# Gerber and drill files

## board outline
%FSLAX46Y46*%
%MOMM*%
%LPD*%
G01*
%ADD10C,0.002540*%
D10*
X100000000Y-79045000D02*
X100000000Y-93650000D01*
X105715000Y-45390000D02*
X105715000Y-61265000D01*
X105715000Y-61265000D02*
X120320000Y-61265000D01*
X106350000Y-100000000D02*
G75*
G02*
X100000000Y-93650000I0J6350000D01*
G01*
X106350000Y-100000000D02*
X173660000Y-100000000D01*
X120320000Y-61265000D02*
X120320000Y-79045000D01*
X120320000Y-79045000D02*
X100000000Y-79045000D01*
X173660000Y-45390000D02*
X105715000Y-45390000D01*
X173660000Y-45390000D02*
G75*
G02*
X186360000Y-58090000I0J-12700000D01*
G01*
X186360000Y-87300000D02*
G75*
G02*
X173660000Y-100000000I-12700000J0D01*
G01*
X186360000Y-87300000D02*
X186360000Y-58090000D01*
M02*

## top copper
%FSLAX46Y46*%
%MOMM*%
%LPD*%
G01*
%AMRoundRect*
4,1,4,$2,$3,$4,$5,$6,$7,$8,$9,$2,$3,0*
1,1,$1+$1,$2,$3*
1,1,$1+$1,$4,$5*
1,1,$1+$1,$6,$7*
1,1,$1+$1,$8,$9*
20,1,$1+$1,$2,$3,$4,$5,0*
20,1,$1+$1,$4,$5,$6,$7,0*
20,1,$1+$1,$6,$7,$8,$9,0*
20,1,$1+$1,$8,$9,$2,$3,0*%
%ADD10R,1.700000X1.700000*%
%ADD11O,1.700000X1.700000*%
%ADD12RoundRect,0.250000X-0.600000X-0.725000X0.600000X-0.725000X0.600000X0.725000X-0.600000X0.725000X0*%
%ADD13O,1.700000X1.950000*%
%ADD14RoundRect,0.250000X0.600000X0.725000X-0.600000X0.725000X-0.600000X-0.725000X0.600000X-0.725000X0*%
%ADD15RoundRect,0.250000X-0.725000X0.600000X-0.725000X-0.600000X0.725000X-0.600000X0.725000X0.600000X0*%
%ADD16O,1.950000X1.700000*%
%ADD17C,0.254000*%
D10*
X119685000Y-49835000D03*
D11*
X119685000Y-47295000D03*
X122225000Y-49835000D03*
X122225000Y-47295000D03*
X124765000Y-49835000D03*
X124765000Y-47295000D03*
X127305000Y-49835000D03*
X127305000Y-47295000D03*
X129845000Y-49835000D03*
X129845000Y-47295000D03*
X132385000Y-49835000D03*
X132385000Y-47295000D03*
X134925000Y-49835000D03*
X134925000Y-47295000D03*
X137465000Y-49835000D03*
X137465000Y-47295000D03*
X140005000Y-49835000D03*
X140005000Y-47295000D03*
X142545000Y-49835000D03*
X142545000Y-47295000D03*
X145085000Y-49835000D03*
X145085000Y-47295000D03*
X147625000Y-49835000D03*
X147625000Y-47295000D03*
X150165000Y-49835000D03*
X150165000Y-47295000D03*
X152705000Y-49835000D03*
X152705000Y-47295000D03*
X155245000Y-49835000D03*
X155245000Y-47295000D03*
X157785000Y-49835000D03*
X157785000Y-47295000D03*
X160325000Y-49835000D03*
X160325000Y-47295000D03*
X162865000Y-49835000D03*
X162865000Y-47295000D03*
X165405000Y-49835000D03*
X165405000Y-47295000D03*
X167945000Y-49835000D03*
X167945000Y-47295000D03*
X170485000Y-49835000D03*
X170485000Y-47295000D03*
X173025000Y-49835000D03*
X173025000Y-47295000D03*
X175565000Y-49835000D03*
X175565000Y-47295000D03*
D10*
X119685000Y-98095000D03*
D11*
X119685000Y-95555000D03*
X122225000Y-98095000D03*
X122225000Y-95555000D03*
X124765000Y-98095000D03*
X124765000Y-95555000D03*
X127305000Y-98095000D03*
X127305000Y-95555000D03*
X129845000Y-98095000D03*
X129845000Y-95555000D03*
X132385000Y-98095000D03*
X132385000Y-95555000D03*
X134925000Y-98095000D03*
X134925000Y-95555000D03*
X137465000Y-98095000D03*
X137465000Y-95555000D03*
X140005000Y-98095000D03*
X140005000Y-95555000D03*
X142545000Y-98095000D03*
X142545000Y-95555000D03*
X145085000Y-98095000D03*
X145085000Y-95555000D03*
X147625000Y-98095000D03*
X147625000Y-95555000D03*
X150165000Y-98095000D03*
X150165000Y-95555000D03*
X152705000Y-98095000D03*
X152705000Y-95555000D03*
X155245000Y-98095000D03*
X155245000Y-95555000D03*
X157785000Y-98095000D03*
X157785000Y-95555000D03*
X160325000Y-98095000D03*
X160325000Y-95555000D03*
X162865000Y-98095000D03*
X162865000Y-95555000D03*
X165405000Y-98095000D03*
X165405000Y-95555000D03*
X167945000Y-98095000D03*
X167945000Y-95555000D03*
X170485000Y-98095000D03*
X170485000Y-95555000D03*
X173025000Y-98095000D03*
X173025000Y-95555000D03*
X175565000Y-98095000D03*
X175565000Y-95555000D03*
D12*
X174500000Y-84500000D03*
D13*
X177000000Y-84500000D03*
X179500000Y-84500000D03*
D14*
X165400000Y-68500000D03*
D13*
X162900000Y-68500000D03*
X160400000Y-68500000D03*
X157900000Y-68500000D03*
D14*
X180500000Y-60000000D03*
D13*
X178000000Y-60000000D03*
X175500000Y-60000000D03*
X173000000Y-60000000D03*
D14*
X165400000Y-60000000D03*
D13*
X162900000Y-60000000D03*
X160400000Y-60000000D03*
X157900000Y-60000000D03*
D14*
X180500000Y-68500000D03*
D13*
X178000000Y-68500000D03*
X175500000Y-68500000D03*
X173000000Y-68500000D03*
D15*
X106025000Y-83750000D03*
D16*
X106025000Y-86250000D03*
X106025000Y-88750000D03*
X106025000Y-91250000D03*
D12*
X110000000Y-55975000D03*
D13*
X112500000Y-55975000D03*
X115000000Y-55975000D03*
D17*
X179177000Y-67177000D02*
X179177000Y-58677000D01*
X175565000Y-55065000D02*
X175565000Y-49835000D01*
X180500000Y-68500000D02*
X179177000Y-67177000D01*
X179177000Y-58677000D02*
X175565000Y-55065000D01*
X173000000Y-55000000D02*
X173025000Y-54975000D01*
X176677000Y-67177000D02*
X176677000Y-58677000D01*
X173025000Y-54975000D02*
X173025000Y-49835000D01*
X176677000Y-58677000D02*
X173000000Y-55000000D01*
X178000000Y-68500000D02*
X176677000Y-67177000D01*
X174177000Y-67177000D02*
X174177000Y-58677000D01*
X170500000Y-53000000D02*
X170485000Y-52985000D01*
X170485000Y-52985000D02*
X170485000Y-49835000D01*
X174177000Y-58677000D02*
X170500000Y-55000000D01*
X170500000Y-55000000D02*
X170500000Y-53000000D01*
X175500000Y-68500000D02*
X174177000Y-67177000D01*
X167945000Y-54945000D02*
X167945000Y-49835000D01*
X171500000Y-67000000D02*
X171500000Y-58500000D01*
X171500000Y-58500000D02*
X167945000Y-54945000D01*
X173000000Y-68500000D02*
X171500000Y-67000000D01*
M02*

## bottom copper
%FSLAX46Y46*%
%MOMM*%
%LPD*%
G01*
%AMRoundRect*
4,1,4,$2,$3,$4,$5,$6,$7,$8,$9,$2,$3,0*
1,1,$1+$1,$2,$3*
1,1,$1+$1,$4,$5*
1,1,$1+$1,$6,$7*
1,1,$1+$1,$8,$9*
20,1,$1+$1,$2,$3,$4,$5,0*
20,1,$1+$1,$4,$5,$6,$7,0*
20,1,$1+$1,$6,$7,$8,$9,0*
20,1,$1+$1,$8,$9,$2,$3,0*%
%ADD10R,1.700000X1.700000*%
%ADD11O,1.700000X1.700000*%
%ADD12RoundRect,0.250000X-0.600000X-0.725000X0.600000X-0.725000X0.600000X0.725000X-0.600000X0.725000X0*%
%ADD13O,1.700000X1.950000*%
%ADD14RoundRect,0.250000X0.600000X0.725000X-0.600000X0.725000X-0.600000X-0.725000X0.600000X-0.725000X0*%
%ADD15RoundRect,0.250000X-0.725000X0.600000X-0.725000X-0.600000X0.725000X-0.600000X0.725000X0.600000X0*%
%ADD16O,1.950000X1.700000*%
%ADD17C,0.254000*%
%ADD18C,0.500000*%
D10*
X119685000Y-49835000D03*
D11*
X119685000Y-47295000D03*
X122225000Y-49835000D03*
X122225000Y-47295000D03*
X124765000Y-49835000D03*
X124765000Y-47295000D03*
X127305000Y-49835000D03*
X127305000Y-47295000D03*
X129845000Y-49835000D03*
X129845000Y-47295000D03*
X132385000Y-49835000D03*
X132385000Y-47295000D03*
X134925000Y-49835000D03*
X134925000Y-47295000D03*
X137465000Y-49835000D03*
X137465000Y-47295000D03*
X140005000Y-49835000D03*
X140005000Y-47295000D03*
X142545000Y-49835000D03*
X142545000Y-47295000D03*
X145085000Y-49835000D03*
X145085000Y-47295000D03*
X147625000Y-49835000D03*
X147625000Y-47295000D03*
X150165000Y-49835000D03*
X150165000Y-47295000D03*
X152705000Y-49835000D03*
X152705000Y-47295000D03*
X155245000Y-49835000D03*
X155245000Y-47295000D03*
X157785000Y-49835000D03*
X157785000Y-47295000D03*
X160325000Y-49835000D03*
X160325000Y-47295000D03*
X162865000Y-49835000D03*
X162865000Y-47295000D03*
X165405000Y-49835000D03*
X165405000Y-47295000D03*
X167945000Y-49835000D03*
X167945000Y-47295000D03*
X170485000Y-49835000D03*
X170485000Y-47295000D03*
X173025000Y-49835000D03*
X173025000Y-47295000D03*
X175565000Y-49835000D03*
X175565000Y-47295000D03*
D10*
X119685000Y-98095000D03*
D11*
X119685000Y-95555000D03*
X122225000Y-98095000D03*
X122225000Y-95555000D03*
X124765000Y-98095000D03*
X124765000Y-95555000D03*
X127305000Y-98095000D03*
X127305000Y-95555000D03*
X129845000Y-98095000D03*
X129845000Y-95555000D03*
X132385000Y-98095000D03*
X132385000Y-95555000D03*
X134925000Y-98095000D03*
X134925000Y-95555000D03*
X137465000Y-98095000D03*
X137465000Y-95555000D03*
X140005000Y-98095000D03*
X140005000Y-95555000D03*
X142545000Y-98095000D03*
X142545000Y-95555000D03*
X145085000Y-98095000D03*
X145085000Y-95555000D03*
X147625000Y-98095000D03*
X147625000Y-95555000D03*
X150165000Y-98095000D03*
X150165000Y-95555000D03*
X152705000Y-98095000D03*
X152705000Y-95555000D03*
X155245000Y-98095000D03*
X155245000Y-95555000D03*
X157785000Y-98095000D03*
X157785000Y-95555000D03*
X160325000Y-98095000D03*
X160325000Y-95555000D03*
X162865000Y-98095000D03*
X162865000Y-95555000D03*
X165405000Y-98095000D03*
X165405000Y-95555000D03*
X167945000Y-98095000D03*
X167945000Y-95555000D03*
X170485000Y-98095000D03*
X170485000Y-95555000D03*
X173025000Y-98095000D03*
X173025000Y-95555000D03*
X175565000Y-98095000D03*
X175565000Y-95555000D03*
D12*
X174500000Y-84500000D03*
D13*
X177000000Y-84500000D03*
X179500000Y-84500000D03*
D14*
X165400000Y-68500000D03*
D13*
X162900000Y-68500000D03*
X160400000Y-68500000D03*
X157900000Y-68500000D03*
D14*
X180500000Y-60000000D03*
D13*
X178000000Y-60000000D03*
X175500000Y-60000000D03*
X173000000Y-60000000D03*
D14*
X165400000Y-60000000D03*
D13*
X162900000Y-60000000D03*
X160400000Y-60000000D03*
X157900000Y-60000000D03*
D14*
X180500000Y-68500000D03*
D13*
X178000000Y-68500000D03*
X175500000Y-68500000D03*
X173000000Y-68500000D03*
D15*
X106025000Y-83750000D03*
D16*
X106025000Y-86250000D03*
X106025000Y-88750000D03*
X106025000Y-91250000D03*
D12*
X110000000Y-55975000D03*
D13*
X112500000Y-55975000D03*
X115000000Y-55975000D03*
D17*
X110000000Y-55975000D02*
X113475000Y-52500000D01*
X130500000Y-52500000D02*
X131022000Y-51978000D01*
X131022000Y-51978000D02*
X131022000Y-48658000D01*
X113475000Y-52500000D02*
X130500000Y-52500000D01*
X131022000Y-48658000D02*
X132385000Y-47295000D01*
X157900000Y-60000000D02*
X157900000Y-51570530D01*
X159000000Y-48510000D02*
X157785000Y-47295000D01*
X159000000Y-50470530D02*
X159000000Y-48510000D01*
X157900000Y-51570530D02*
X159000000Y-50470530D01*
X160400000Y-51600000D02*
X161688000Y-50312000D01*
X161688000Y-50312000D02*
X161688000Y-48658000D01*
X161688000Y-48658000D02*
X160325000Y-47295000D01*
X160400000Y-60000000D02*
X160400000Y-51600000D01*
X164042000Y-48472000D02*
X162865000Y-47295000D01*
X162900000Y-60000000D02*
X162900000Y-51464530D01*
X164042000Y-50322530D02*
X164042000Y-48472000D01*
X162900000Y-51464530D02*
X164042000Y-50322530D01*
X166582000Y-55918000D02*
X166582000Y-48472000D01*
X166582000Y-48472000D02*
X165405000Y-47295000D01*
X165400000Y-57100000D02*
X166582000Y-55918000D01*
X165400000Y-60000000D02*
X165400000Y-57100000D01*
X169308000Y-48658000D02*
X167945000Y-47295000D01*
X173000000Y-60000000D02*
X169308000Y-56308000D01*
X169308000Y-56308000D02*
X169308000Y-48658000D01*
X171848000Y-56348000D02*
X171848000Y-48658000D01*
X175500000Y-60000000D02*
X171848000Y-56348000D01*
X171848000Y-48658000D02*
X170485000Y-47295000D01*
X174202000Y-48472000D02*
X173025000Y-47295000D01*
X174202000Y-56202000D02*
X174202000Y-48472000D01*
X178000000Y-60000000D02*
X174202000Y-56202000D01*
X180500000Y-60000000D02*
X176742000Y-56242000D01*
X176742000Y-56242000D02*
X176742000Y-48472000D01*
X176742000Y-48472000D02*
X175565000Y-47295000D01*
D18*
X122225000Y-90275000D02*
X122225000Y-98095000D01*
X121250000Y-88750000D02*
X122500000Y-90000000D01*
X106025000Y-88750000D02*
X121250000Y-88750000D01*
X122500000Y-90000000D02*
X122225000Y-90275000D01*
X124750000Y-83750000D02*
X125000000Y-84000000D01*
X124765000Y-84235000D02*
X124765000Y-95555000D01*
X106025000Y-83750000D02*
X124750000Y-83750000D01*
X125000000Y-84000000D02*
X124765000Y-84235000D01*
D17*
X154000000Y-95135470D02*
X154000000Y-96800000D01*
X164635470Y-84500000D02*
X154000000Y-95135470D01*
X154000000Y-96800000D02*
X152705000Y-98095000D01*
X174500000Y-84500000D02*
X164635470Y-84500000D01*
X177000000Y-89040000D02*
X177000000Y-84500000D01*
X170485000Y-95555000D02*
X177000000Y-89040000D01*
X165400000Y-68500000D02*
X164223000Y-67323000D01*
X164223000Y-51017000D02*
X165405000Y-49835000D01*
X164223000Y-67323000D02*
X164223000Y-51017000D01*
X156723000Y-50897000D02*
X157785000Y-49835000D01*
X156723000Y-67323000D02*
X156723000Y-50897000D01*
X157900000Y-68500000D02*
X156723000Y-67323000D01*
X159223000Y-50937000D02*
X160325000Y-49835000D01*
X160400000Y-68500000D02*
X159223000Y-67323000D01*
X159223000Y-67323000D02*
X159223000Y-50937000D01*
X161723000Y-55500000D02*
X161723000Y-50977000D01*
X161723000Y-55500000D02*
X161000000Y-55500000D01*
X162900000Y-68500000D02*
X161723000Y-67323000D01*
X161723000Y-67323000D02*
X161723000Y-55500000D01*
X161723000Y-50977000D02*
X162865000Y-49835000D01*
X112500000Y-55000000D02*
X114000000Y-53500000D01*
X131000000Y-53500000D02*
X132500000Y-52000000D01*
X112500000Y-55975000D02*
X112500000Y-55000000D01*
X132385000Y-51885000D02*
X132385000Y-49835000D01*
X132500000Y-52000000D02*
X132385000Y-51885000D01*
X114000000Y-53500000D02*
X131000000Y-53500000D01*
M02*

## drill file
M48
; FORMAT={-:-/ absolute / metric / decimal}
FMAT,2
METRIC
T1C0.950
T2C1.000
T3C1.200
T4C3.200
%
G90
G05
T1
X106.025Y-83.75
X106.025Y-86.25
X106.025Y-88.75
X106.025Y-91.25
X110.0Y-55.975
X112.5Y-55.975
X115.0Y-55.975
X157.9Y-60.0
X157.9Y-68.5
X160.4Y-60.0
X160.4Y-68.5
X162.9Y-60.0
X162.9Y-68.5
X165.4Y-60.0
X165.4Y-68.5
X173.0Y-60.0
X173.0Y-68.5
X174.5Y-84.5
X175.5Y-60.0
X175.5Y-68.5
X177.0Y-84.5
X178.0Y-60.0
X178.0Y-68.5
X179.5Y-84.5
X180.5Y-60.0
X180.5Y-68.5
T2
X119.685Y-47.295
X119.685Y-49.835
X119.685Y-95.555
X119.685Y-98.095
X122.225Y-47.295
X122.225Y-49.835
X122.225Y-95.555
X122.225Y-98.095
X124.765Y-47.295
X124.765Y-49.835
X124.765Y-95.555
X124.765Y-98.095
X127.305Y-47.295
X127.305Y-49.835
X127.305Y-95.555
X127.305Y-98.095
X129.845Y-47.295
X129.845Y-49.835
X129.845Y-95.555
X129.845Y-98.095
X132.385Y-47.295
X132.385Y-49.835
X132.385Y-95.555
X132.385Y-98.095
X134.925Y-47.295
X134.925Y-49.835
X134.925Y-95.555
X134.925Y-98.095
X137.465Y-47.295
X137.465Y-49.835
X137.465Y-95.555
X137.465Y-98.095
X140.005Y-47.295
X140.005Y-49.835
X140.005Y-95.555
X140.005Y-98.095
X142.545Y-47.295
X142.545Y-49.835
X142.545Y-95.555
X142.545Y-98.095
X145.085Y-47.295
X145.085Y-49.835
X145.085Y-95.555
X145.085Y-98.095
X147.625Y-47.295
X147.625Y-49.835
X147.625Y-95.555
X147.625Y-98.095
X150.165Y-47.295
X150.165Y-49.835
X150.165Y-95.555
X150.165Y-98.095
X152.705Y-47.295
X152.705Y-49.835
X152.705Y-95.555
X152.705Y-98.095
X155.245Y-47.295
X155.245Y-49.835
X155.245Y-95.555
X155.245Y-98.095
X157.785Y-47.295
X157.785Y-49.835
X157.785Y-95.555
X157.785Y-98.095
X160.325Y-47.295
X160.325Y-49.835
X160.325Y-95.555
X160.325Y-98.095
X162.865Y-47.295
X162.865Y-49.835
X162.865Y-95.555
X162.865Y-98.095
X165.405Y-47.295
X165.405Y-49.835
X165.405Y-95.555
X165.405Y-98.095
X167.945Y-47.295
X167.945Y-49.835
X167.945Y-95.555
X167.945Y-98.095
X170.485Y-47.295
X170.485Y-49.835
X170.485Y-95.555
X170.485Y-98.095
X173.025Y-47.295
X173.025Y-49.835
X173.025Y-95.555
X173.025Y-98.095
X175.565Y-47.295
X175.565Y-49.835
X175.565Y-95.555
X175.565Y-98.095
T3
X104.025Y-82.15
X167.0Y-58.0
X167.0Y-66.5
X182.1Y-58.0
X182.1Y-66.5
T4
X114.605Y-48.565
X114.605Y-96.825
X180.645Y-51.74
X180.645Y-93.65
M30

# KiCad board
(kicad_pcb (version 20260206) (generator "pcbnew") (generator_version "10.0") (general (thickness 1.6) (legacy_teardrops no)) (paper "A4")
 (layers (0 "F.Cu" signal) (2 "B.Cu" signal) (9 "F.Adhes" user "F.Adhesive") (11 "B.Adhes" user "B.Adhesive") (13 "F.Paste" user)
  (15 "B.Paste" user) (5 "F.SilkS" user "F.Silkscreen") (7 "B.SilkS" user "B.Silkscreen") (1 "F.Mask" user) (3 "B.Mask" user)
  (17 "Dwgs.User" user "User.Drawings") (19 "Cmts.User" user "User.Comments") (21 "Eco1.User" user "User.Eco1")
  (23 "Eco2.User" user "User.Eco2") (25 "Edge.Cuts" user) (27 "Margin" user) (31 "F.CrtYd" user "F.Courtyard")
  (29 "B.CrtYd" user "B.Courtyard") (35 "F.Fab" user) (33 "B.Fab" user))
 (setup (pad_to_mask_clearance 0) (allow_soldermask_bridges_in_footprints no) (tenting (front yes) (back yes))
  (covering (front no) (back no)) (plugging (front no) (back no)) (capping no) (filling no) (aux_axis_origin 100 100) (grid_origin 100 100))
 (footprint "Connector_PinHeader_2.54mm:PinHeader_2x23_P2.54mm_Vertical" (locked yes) (layer "F.Cu") (at 119.685 49.835 90)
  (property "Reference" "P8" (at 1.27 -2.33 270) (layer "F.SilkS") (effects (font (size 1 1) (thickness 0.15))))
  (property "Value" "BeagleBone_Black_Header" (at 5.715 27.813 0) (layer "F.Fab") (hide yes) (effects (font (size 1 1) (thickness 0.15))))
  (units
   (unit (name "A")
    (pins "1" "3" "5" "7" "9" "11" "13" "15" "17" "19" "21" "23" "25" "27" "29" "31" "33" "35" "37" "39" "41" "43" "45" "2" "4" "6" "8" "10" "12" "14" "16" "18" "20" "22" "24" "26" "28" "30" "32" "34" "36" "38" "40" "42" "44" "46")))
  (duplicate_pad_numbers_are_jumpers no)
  (pad "1" thru_hole rect (at 0 0 90) (size 1.7 1.7) (drill 1) (layers "*.Cu" "*.Mask") (remove_unused_layers no) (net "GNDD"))
  (pad "2" thru_hole oval (at 2.54 0 90) (size 1.7 1.7) (drill 1) (layers "*.Cu" "*.Mask") (remove_unused_layers no) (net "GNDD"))
  (pad "3" thru_hole oval (at 0 2.54 90) (size 1.7 1.7) (drill 1) (layers "*.Cu" "*.Mask") (remove_unused_layers no)
   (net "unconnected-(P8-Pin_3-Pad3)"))
  (pad "4" thru_hole oval (at 2.54 2.54 90) (size 1.7 1.7) (drill 1) (layers "*.Cu" "*.Mask") (remove_unused_layers no) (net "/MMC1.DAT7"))
  (pad "5" thru_hole oval (at 0 5.08 90) (size 1.7 1.7) (drill 1) (layers "*.Cu" "*.Mask") (remove_unused_layers no)
   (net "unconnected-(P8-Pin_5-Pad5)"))
  (pad "6" thru_hole oval (at 2.54 5.08 90) (size 1.7 1.7) (drill 1) (layers "*.Cu" "*.Mask") (remove_unused_layers no) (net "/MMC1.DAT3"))
  (pad "7" thru_hole oval (at 0 7.62 90) (size 1.7 1.7) (drill 1) (layers "*.Cu" "*.Mask") (remove_unused_layers no)
   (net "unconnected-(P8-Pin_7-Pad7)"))
  (pad "8" thru_hole oval (at 2.54 7.62 90) (size 1.7 1.7) (drill 1) (layers "*.Cu" "*.Mask") (remove_unused_layers no) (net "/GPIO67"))
  (pad "9" thru_hole oval (at 0 10.16 90) (size 1.7 1.7) (drill 1) (layers "*.Cu" "*.Mask") (remove_unused_layers no)
   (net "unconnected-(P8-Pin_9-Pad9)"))
  (pad "10" thru_hole oval (at 2.54 10.16 90) (size 1.7 1.7) (drill 1) (layers "*.Cu" "*.Mask") (remove_unused_layers no) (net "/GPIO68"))
  (pad "11" thru_hole oval (at 0 12.7 90) (size 1.7 1.7) (drill 1) (layers "*.Cu" "*.Mask") (remove_unused_layers no) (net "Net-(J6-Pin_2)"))
  (pad "12" thru_hole oval (at 2.54 12.7 90) (size 1.7 1.7) (drill 1) (layers "*.Cu" "*.Mask") (remove_unused_layers no) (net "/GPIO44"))
  (pad "13" thru_hole oval (at 0 15.24 90) (size 1.7 1.7) (drill 1) (layers "*.Cu" "*.Mask") (remove_unused_layers no)
   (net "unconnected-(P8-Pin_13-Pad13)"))
  (pad "14" thru_hole oval (at 2.54 15.24 90) (size 1.7 1.7) (drill 1) (layers "*.Cu" "*.Mask") (remove_unused_layers no) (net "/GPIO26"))
  (pad "15" thru_hole oval (at 0 17.78 90) (size 1.7 1.7) (drill 1) (layers "*.Cu" "*.Mask") (remove_unused_layers no)
   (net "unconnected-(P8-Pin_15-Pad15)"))
  (pad "16" thru_hole oval (at 2.54 17.78 90) (size 1.7 1.7) (drill 1) (layers "*.Cu" "*.Mask") (remove_unused_layers no) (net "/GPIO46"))
  (pad "17" thru_hole oval (at 0 20.32 90) (size 1.7 1.7) (drill 1) (layers "*.Cu" "*.Mask") (remove_unused_layers no)
   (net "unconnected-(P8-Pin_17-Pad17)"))
  (pad "18" thru_hole oval (at 2.54 20.32 90) (size 1.7 1.7) (drill 1) (layers "*.Cu" "*.Mask") (remove_unused_layers no) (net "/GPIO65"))
  (pad "19" thru_hole oval (at 0 22.86 90) (size 1.7 1.7) (drill 1) (layers "*.Cu" "*.Mask") (remove_unused_layers no)
   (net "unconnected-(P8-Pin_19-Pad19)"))
  (pad "20" thru_hole oval (at 2.54 22.86 90) (size 1.7 1.7) (drill 1) (layers "*.Cu" "*.Mask") (remove_unused_layers no) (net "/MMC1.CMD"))
  (pad "21" thru_hole oval (at 0 25.4 90) (size 1.7 1.7) (drill 1) (layers "*.Cu" "*.Mask") (remove_unused_layers no)
   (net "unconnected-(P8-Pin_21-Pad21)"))
  (pad "22" thru_hole oval (at 2.54 25.4 90) (size 1.7 1.7) (drill 1) (layers "*.Cu" "*.Mask") (remove_unused_layers no) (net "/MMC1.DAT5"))
  (pad "23" thru_hole oval (at 0 27.94 90) (size 1.7 1.7) (drill 1) (layers "*.Cu" "*.Mask") (remove_unused_layers no)
   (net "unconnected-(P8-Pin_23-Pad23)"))
  (pad "24" thru_hole oval (at 2.54 27.94 90) (size 1.7 1.7) (drill 1) (layers "*.Cu" "*.Mask") (remove_unused_layers no) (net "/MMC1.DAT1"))
  (pad "25" thru_hole oval (at 0 30.48 90) (size 1.7 1.7) (drill 1) (layers "*.Cu" "*.Mask") (remove_unused_layers no)
   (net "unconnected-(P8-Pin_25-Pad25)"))
  (pad "26" thru_hole oval (at 2.54 30.48 90) (size 1.7 1.7) (drill 1) (layers "*.Cu" "*.Mask") (remove_unused_layers no) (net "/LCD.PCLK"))
  (pad "27" thru_hole oval (at 0 33.02 90) (size 1.7 1.7) (drill 1) (layers "*.Cu" "*.Mask") (remove_unused_layers no)
   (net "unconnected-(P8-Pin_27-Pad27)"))
  (pad "28" thru_hole oval (at 2.54 33.02 90) (size 1.7 1.7) (drill 1) (layers "*.Cu" "*.Mask") (remove_unused_layers no) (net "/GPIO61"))
  (pad "29" thru_hole oval (at 0 35.56 90) (size 1.7 1.7) (drill 1) (layers "*.Cu" "*.Mask") (remove_unused_layers no)
   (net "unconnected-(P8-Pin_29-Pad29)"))
  (pad "30" thru_hole oval (at 2.54 35.56 90) (size 1.7 1.7) (drill 1) (layers "*.Cu" "*.Mask") (remove_unused_layers no)
   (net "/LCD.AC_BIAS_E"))
  (pad "31" thru_hole oval (at 0 38.1 90) (size 1.7 1.7) (drill 1) (layers "*.Cu" "*.Mask") (remove_unused_layers no) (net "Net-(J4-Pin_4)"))
  (pad "32" thru_hole oval (at 2.54 38.1 90) (size 1.7 1.7) (drill 1) (layers "*.Cu" "*.Mask") (remove_unused_layers no) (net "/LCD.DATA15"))
  (pad "33" thru_hole oval (at 0 40.64 90) (size 1.7 1.7) (drill 1) (layers "*.Cu" "*.Mask") (remove_unused_layers no)
   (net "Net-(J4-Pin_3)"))
  (pad "34" thru_hole oval (at 2.54 40.64 90) (size 1.7 1.7) (drill 1) (layers "*.Cu" "*.Mask") (remove_unused_layers no)
   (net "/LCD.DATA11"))
  (pad "35" thru_hole oval (at 0 43.18 90) (size 1.7 1.7) (drill 1) (layers "*.Cu" "*.Mask") (remove_unused_layers no)
   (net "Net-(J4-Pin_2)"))
  (pad "36" thru_hole oval (at 2.54 43.18 90) (size 1.7 1.7) (drill 1) (layers "*.Cu" "*.Mask") (remove_unused_layers no)
   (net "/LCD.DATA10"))
  (pad "37" thru_hole oval (at 0 45.72 90) (size 1.7 1.7) (drill 1) (layers "*.Cu" "*.Mask") (remove_unused_layers no)
   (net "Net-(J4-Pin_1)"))
  (pad "38" thru_hole oval (at 2.54 45.72 90) (size 1.7 1.7) (drill 1) (layers "*.Cu" "*.Mask") (remove_unused_layers no) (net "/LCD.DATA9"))
  (pad "39" thru_hole oval (at 0 48.26 90) (size 1.7 1.7) (drill 1) (layers "*.Cu" "*.Mask") (remove_unused_layers no)
   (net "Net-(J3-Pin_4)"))
  (pad "40" thru_hole oval (at 2.54 48.26 90) (size 1.7 1.7) (drill 1) (layers "*.Cu" "*.Mask") (remove_unused_layers no) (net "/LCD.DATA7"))
  (pad "41" thru_hole oval (at 0 50.8 90) (size 1.7 1.7) (drill 1) (layers "*.Cu" "*.Mask") (remove_unused_layers no) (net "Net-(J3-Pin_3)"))
  (pad "42" thru_hole oval (at 2.54 50.8 90) (size 1.7 1.7) (drill 1) (layers "*.Cu" "*.Mask") (remove_unused_layers no) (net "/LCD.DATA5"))
  (pad "43" thru_hole oval (at 0 53.34 90) (size 1.7 1.7) (drill 1) (layers "*.Cu" "*.Mask") (remove_unused_layers no)
   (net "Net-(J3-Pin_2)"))
  (pad "44" thru_hole oval (at 2.54 53.34 90) (size 1.7 1.7) (drill 1) (layers "*.Cu" "*.Mask") (remove_unused_layers no) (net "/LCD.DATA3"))
  (pad "45" thru_hole oval (at 0 55.88 90) (size 1.7 1.7) (drill 1) (layers "*.Cu" "*.Mask") (remove_unused_layers no)
   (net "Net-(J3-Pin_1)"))
  (pad "46" thru_hole oval (at 2.54 55.88 90) (size 1.7 1.7) (drill 1) (layers "*.Cu" "*.Mask") (remove_unused_layers no) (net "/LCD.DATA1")))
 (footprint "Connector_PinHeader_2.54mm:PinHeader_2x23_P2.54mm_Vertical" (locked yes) (layer "F.Cu") (at 119.685 98.095 90)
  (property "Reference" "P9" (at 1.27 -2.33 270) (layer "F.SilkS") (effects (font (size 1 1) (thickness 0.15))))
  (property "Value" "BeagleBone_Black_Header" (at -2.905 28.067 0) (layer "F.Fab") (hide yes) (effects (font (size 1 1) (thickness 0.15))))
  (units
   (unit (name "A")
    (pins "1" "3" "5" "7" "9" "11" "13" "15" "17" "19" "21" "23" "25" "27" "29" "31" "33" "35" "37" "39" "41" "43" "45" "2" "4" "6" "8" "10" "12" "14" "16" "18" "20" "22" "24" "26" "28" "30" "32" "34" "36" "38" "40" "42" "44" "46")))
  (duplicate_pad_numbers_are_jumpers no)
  (pad "1" thru_hole rect (at 0 0 90) (size 1.7 1.7) (drill 1) (layers "*.Cu" "*.Mask") (remove_unused_layers no) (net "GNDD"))
  (pad "2" thru_hole oval (at 2.54 0 90) (size 1.7 1.7) (drill 1) (layers "*.Cu" "*.Mask") (remove_unused_layers no) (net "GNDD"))
  (pad "3" thru_hole oval (at 0 2.54 90) (size 1.7 1.7) (drill 1) (layers "*.Cu" "*.Mask") (remove_unused_layers no) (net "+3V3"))
  (pad "4" thru_hole oval (at 2.54 2.54 90) (size 1.7 1.7) (drill 1) (layers "*.Cu" "*.Mask") (remove_unused_layers no) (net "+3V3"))
  (pad "5" thru_hole oval (at 0 5.08 90) (size 1.7 1.7) (drill 1) (layers "*.Cu" "*.Mask") (remove_unused_layers no) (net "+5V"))
  (pad "6" thru_hole oval (at 2.54 5.08 90) (size 1.7 1.7) (drill 1) (layers "*.Cu" "*.Mask") (remove_unused_layers no) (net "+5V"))
  (pad "7" thru_hole oval (at 0 7.62 90) (size 1.7 1.7) (drill 1) (layers "*.Cu" "*.Mask") (remove_unused_layers no) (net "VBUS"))
  (pad "8" thru_hole oval (at 2.54 7.62 90) (size 1.7 1.7) (drill 1) (layers "*.Cu" "*.Mask") (remove_unused_layers no) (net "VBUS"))
  (pad "9" thru_hole oval (at 0 10.16 90) (size 1.7 1.7) (drill 1) (layers "*.Cu" "*.Mask") (remove_unused_layers no) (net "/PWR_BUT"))
  (pad "10" thru_hole oval (at 2.54 10.16 90) (size 1.7 1.7) (drill 1) (layers "*.Cu" "*.Mask") (remove_unused_layers no)
   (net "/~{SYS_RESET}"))
  (pad "11" thru_hole oval (at 0 12.7 90) (size 1.7 1.7) (drill 1) (layers "*.Cu" "*.Mask") (remove_unused_layers no) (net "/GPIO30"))
  (pad "12" thru_hole oval (at 2.54 12.7 90) (size 1.7 1.7) (drill 1) (layers "*.Cu" "*.Mask") (remove_unused_layers no) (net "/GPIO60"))
  (pad "13" thru_hole oval (at 0 15.24 90) (size 1.7 1.7) (drill 1) (layers "*.Cu" "*.Mask") (remove_unused_layers no) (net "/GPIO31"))
  (pad "14" thru_hole oval (at 2.54 15.24 90) (size 1.7 1.7) (drill 1) (layers "*.Cu" "*.Mask") (remove_unused_layers no) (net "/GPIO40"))
  (pad "15" thru_hole oval (at 0 17.78 90) (size 1.7 1.7) (drill 1) (layers "*.Cu" "*.Mask") (remove_unused_layers no) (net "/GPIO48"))
  (pad "16" thru_hole oval (at 2.54 17.78 90) (size 1.7 1.7) (drill 1) (layers "*.Cu" "*.Mask") (remove_unused_layers no) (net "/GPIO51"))
  (pad "17" thru_hole oval (at 0 20.32 90) (size 1.7 1.7) (drill 1) (layers "*.Cu" "*.Mask") (remove_unused_layers no) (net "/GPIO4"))
  (pad "18" thru_hole oval (at 2.54 20.32 90) (size 1.7 1.7) (drill 1) (layers "*.Cu" "*.Mask") (remove_unused_layers no) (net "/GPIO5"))
  (pad "19" thru_hole oval (at 0 22.86 90) (size 1.7 1.7) (drill 1) (layers "*.Cu" "*.Mask") (remove_unused_layers no) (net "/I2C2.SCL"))
  (pad "20" thru_hole oval (at 2.54 22.86 90) (size 1.7 1.7) (drill 1) (layers "*.Cu" "*.Mask") (remove_unused_layers no) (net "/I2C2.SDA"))
  (pad "21" thru_hole oval (at 0 25.4 90) (size 1.7 1.7) (drill 1) (layers "*.Cu" "*.Mask") (remove_unused_layers no) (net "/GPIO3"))
  (pad "22" thru_hole oval (at 2.54 25.4 90) (size 1.7 1.7) (drill 1) (layers "*.Cu" "*.Mask") (remove_unused_layers no) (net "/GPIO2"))
  (pad "23" thru_hole oval (at 0 27.94 90) (size 1.7 1.7) (drill 1) (layers "*.Cu" "*.Mask") (remove_unused_layers no) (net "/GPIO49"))
  (pad "24" thru_hole oval (at 2.54 27.94 90) (size 1.7 1.7) (drill 1) (layers "*.Cu" "*.Mask") (remove_unused_layers no) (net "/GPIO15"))
  (pad "25" thru_hole oval (at 0 30.48 90) (size 1.7 1.7) (drill 1) (layers "*.Cu" "*.Mask") (remove_unused_layers no) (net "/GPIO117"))
  (pad "26" thru_hole oval (at 2.54 30.48 90) (size 1.7 1.7) (drill 1) (layers "*.Cu" "*.Mask") (remove_unused_layers no) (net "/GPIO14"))
  (pad "27" thru_hole oval (at 0 33.02 90) (size 1.7 1.7) (drill 1) (layers "*.Cu" "*.Mask") (remove_unused_layers no) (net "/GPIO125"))
  (pad "28" thru_hole oval (at 2.54 33.02 90) (size 1.7 1.7) (drill 1) (layers "*.Cu" "*.Mask") (remove_unused_layers no) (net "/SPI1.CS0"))
  (pad "29" thru_hole oval (at 0 35.56 90) (size 1.7 1.7) (drill 1) (layers "*.Cu" "*.Mask") (remove_unused_layers no) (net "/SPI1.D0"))
  (pad "30" thru_hole oval (at 2.54 35.56 90) (size 1.7 1.7) (drill 1) (layers "*.Cu" "*.Mask") (remove_unused_layers no) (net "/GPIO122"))
  (pad "31" thru_hole oval (at 0 38.1 90) (size 1.7 1.7) (drill 1) (layers "*.Cu" "*.Mask") (remove_unused_layers no) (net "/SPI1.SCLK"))
  (pad "32" thru_hole oval (at 2.54 38.1 90) (size 1.7 1.7) (drill 1) (layers "*.Cu" "*.Mask") (remove_unused_layers no) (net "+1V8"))
  (pad "33" thru_hole oval (at 0 40.64 90) (size 1.7 1.7) (drill 1) (layers "*.Cu" "*.Mask") (remove_unused_layers no) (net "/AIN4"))
  (pad "34" thru_hole oval (at 2.54 40.64 90) (size 1.7 1.7) (drill 1) (layers "*.Cu" "*.Mask") (remove_unused_layers no) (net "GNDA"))
  (pad "35" thru_hole oval (at 0 43.18 90) (size 1.7 1.7) (drill 1) (layers "*.Cu" "*.Mask") (remove_unused_layers no) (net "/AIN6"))
  (pad "36" thru_hole oval (at 2.54 43.18 90) (size 1.7 1.7) (drill 1) (layers "*.Cu" "*.Mask") (remove_unused_layers no) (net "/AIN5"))
  (pad "37" thru_hole oval (at 0 45.72 90) (size 1.7 1.7) (drill 1) (layers "*.Cu" "*.Mask") (remove_unused_layers no) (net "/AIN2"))
  (pad "38" thru_hole oval (at 2.54 45.72 90) (size 1.7 1.7) (drill 1) (layers "*.Cu" "*.Mask") (remove_unused_layers no) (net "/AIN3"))
  (pad "39" thru_hole oval (at 0 48.26 90) (size 1.7 1.7) (drill 1) (layers "*.Cu" "*.Mask") (remove_unused_layers no) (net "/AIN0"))
  (pad "40" thru_hole oval (at 2.54 48.26 90) (size 1.7 1.7) (drill 1) (layers "*.Cu" "*.Mask") (remove_unused_layers no) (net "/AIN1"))
  (pad "41" thru_hole oval (at 0 50.8 90) (size 1.7 1.7) (drill 1) (layers "*.Cu" "*.Mask") (remove_unused_layers no) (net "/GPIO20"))
  (pad "42" thru_hole oval (at 2.54 50.8 90) (size 1.7 1.7) (drill 1) (layers "*.Cu" "*.Mask") (remove_unused_layers no) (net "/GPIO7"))
  (pad "43" thru_hole oval (at 0 53.34 90) (size 1.7 1.7) (drill 1) (layers "*.Cu" "*.Mask") (remove_unused_layers no) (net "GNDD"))
  (pad "44" thru_hole oval (at 2.54 53.34 90) (size 1.7 1.7) (drill 1) (layers "*.Cu" "*.Mask") (remove_unused_layers no) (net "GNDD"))
  (pad "45" thru_hole oval (at 0 55.88 90) (size 1.7 1.7) (drill 1) (layers "*.Cu" "*.Mask") (remove_unused_layers no) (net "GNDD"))
  (pad "46" thru_hole oval (at 2.54 55.88 90) (size 1.7 1.7) (drill 1) (layers "*.Cu" "*.Mask") (remove_unused_layers no) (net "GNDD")))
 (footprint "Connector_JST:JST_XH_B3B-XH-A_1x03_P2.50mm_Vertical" (layer "F.Cu") (at 174.5 84.5)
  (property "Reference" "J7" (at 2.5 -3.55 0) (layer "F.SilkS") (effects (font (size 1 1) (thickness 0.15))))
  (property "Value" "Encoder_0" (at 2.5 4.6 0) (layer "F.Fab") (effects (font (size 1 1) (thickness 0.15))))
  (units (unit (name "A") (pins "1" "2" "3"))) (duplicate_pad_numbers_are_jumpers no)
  (pad "1" thru_hole roundrect (at 0 0) (size 1.7 1.95) (drill 0.95) (layers "*.Cu" "*.Mask") (remove_unused_layers no)
   (roundrect_rratio 0.147059) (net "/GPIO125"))
  (pad "2" thru_hole oval (at 2.5 0) (size 1.7 1.95) (drill 0.95) (layers "*.Cu" "*.Mask") (remove_unused_layers no) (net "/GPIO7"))
  (pad "3" thru_hole oval (at 5 0) (size 1.7 1.95) (drill 0.95) (layers "*.Cu" "*.Mask") (remove_unused_layers no)
   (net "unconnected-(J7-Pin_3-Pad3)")))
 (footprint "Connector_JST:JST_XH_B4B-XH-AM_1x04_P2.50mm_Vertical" (layer "F.Cu") (at 165.4 68.5 180)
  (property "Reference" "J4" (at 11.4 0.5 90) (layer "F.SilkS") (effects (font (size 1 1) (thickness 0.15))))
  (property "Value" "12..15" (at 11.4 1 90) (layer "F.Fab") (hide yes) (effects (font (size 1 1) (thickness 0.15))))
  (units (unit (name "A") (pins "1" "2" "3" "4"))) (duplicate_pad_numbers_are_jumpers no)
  (pad "" np_thru_hole circle (at -1.6 2 180) (size 1.2 1.2) (drill 1.2) (layers "*.Cu" "*.Mask"))
  (pad "1" thru_hole roundrect (at 0 0 180) (size 1.7 1.95) (drill 0.95) (layers "*.Cu" "*.Mask") (remove_unused_layers no)
   (roundrect_rratio 0.147059) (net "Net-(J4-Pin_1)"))
  (pad "2" thru_hole oval (at 2.5 0 180) (size 1.7 1.95) (drill 0.95) (layers "*.Cu" "*.Mask") (remove_unused_layers no)
   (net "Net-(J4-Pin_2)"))
  (pad "3" thru_hole oval (at 5 0 180) (size 1.7 1.95) (drill 0.95) (layers "*.Cu" "*.Mask") (remove_unused_layers no)
   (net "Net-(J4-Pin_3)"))
  (pad "4" thru_hole oval (at 7.5 0 180) (size 1.7 1.95) (drill 0.95) (layers "*.Cu" "*.Mask") (remove_unused_layers no)
   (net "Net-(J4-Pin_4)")))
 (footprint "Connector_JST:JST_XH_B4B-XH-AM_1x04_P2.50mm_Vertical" (layer "F.Cu") (at 180.5 60 180)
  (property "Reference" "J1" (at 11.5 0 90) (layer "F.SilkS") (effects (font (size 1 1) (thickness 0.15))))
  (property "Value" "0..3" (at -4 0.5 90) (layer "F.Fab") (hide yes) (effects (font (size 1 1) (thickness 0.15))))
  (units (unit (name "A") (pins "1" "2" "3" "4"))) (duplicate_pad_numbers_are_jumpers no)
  (pad "" np_thru_hole circle (at -1.6 2 180) (size 1.2 1.2) (drill 1.2) (layers "*.Cu" "*.Mask"))
  (pad "1" thru_hole roundrect (at 0 0 180) (size 1.7 1.95) (drill 0.95) (layers "*.Cu" "*.Mask") (remove_unused_layers no)
   (roundrect_rratio 0.147059) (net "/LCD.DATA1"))
  (pad "2" thru_hole oval (at 2.5 0 180) (size 1.7 1.95) (drill 0.95) (layers "*.Cu" "*.Mask") (remove_unused_layers no) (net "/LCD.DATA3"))
  (pad "3" thru_hole oval (at 5 0 180) (size 1.7 1.95) (drill 0.95) (layers "*.Cu" "*.Mask") (remove_unused_layers no) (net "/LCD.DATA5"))
  (pad "4" thru_hole oval (at 7.5 0 180) (size 1.7 1.95) (drill 0.95) (layers "*.Cu" "*.Mask") (remove_unused_layers no) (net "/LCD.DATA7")))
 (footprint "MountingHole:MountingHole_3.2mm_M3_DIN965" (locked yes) (layer "F.Cu") (at 180.645 51.74)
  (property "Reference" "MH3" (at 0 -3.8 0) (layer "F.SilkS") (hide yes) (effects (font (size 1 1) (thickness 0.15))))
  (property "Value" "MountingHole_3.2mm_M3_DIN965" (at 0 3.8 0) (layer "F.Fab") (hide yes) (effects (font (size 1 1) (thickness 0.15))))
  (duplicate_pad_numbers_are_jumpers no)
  (pad "" np_thru_hole circle (at 0 0) (size 3.2 3.2) (drill 3.2) (layers "*.Cu" "*.Mask")))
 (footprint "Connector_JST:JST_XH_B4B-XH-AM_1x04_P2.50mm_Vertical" (layer "F.Cu") (at 165.4 60 180)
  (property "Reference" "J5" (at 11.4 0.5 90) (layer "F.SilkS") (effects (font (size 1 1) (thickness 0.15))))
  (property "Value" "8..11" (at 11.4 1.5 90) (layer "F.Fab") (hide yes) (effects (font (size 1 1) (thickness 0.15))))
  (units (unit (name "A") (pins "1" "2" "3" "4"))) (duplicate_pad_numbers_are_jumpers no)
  (pad "" np_thru_hole circle (at -1.6 2 180) (size 1.2 1.2) (drill 1.2) (layers "*.Cu" "*.Mask"))
  (pad "1" thru_hole roundrect (at 0 0 180) (size 1.7 1.95) (drill 0.95) (layers "*.Cu" "*.Mask") (remove_unused_layers no)
   (roundrect_rratio 0.147059) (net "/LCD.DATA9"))
  (pad "2" thru_hole oval (at 2.5 0 180) (size 1.7 1.95) (drill 0.95) (layers "*.Cu" "*.Mask") (remove_unused_layers no) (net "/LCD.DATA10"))
  (pad "3" thru_hole oval (at 5 0 180) (size 1.7 1.95) (drill 0.95) (layers "*.Cu" "*.Mask") (remove_unused_layers no) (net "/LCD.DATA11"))
  (pad "4" thru_hole oval (at 7.5 0 180) (size 1.7 1.95) (drill 0.95) (layers "*.Cu" "*.Mask") (remove_unused_layers no) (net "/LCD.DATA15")))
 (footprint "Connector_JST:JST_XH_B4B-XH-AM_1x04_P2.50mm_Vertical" (layer "F.Cu") (at 180.5 68.5 180)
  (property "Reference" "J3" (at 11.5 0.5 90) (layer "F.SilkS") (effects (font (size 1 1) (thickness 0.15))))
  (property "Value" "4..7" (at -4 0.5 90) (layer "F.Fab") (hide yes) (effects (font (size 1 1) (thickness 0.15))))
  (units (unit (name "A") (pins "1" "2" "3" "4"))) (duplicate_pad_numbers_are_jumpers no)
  (pad "" np_thru_hole circle (at -1.6 2 180) (size 1.2 1.2) (drill 1.2) (layers "*.Cu" "*.Mask"))
  (pad "1" thru_hole roundrect (at 0 0 180) (size 1.7 1.95) (drill 0.95) (layers "*.Cu" "*.Mask") (remove_unused_layers no)
   (roundrect_rratio 0.147059) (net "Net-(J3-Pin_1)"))
  (pad "2" thru_hole oval (at 2.5 0 180) (size 1.7 1.95) (drill 0.95) (layers "*.Cu" "*.Mask") (remove_unused_layers no)
   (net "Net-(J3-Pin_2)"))
  (pad "3" thru_hole oval (at 5 0 180) (size 1.7 1.95) (drill 0.95) (layers "*.Cu" "*.Mask") (remove_unused_layers no)
   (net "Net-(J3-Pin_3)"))
  (pad "4" thru_hole oval (at 7.5 0 180) (size 1.7 1.95) (drill 0.95) (layers "*.Cu" "*.Mask") (remove_unused_layers no)
   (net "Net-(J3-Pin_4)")))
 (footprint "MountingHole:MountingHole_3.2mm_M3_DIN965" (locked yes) (layer "F.Cu") (at 180.645 93.65)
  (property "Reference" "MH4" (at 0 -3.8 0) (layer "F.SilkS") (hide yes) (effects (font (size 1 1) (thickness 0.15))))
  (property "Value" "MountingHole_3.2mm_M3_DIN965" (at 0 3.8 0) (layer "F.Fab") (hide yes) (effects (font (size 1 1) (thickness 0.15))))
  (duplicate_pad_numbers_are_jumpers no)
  (pad "" np_thru_hole circle (at 0 0) (size 3.2 3.2) (drill 3.2) (layers "*.Cu" "*.Mask")))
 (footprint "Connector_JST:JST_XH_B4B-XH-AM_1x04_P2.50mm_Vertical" (layer "F.Cu") (at 106.025 83.75 -90)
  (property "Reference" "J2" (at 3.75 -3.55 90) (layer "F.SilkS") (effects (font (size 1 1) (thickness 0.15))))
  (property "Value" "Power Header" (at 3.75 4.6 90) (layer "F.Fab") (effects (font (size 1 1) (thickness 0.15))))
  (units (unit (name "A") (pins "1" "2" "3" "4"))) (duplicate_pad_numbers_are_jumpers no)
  (pad "" np_thru_hole circle (at -1.6 2 270) (size 1.2 1.2) (drill 1.2) (layers "*.Cu" "*.Mask"))
  (pad "1" thru_hole roundrect (at 0 0 270) (size 1.7 1.95) (drill 0.95) (layers "*.Cu" "*.Mask") (remove_unused_layers no)
   (roundrect_rratio 0.147059) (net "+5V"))
  (pad "2" thru_hole oval (at 2.5 0 270) (size 1.7 1.95) (drill 0.95) (layers "*.Cu" "*.Mask") (remove_unused_layers no) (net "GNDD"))
  (pad "3" thru_hole oval (at 5 0 270) (size 1.7 1.95) (drill 0.95) (layers "*.Cu" "*.Mask") (remove_unused_layers no) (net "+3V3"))
  (pad "4" thru_hole oval (at 7.5 0 270) (size 1.7 1.95) (drill 0.95) (layers "*.Cu" "*.Mask") (remove_unused_layers no) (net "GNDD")))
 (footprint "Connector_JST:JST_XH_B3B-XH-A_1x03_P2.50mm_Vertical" (layer "F.Cu") (at 110 55.975)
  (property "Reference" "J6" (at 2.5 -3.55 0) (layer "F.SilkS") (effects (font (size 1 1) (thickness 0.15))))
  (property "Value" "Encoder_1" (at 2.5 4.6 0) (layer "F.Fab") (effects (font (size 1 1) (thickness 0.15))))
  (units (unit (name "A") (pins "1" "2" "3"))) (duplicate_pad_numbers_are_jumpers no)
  (pad "1" thru_hole roundrect (at 0 0) (size 1.7 1.95) (drill 0.95) (layers "*.Cu" "*.Mask") (remove_unused_layers no)
   (roundrect_rratio 0.147059) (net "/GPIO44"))
  (pad "2" thru_hole oval (at 2.5 0) (size 1.7 1.95) (drill 0.95) (layers "*.Cu" "*.Mask") (remove_unused_layers no) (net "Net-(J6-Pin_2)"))
  (pad "3" thru_hole oval (at 5 0) (size 1.7 1.95) (drill 0.95) (layers "*.Cu" "*.Mask") (remove_unused_layers no)
   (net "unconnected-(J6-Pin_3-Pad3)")))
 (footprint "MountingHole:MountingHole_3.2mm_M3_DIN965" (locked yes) (layer "F.Cu") (at 114.605 48.565)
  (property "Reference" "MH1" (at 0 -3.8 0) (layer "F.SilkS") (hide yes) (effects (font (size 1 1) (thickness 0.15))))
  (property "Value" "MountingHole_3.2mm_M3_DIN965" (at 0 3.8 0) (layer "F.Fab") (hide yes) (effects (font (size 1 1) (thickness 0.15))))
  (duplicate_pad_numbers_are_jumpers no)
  (pad "" np_thru_hole circle (at 0 0) (size 3.2 3.2) (drill 3.2) (layers "*.Cu" "*.Mask")))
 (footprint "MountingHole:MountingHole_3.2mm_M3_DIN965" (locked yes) (layer "F.Cu") (at 114.605 96.825)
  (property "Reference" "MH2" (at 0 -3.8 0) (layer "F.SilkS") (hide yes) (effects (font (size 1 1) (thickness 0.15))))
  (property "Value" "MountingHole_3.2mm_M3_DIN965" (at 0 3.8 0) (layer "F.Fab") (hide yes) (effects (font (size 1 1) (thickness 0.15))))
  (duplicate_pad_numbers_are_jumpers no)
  (pad "" np_thru_hole circle (at 0 0) (size 3.2 3.2) (drill 3.2) (layers "*.Cu" "*.Mask")))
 (gr_line (start 100 79.045) (end 100 93.65) (stroke (width 0.00254) (type solid)) (locked yes) (layer "Edge.Cuts"))
 (gr_line (start 105.715 45.39) (end 105.715 61.265) (stroke (width 0.00254) (type solid)) (locked yes) (layer "Edge.Cuts"))
 (gr_line (start 105.715 61.265) (end 120.32 61.265) (stroke (width 0.00254) (type solid)) (locked yes) (layer "Edge.Cuts"))
 (gr_arc (start 106.35 100) (mid 101.859872 98.140128) (end 100 93.65) (stroke (width 0.00254) (type solid)) (locked yes)
  (layer "Edge.Cuts"))
 (gr_line (start 106.35 100) (end 173.66 100) (stroke (width 0.00254) (type solid)) (locked yes) (layer "Edge.Cuts"))
 (gr_line (start 120.32 61.265) (end 120.32 79.045) (stroke (width 0.00254) (type solid)) (locked yes) (layer "Edge.Cuts"))
 (gr_line (start 120.32 79.045) (end 100 79.045) (stroke (width 0.00254) (type solid)) (locked yes) (layer "Edge.Cuts"))
 (gr_line (start 173.66 45.39) (end 105.715 45.39) (stroke (width 0.00254) (type solid)) (locked yes) (layer "Edge.Cuts"))
 (gr_arc (start 173.66 45.39) (mid 182.640256 49.109744) (end 186.36 58.09) (stroke (width 0.00254) (type solid)) (locked yes)
  (layer "Edge.Cuts"))
 (gr_arc (start 186.36 87.3) (mid 182.640256 96.280256) (end 173.66 100) (stroke (width 0.00254) (type solid)) (locked yes)
  (layer "Edge.Cuts"))
 (gr_line (start 186.36 87.3) (end 186.36 58.09) (stroke (width 0.00254) (type solid)) (locked yes) (layer "Edge.Cuts"))
 (segment (start 110 55.975) (end 113.475 52.5) (width 0.254) (layer "B.Cu") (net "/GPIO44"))
 (segment (start 130.5 52.5) (end 131.022 51.978) (width 0.254) (layer "B.Cu") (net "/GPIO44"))
 (segment (start 131.022 51.978) (end 131.022 48.658) (width 0.254) (layer "B.Cu") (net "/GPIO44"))
 (segment (start 113.475 52.5) (end 130.5 52.5) (width 0.254) (layer "B.Cu") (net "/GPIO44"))
 (segment (start 131.022 48.658) (end 132.385 47.295) (width 0.254) (layer "B.Cu") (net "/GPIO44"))
 (segment (start 157.9 60) (end 157.9 51.57053) (width 0.254) (layer "B.Cu") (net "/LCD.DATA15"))
 (segment (start 159 48.51) (end 157.785 47.295) (width 0.254) (layer "B.Cu") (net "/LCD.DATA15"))
 (segment (start 159 50.47053) (end 159 48.51) (width 0.254) (layer "B.Cu") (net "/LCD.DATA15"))
 (segment (start 157.9 51.57053) (end 159 50.47053) (width 0.254) (layer "B.Cu") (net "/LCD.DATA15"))
 (segment (start 160.4 51.6) (end 161.688 50.312) (width 0.254) (layer "B.Cu") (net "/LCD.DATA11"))
 (segment (start 161.688 50.312) (end 161.688 48.658) (width 0.254) (layer "B.Cu") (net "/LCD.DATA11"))
 (segment (start 161.688 48.658) (end 160.325 47.295) (width 0.254) (layer "B.Cu") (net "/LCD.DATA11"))
 (segment (start 160.4 60) (end 160.4 51.6) (width 0.254) (layer "B.Cu") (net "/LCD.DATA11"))
 (segment (start 164.042 48.472) (end 162.865 47.295) (width 0.254) (layer "B.Cu") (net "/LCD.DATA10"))
 (segment (start 162.9 60) (end 162.9 51.46453) (width 0.254) (layer "B.Cu") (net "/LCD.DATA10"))
 (segment (start 164.042 50.32253) (end 164.042 48.472) (width 0.254) (layer "B.Cu") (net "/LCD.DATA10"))
 (segment (start 162.9 51.46453) (end 164.042 50.32253) (width 0.254) (layer "B.Cu") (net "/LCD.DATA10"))
 (segment (start 166.582 55.918) (end 166.582 48.472) (width 0.254) (layer "B.Cu") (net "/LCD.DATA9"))
 (segment (start 166.582 48.472) (end 165.405 47.295) (width 0.254) (layer "B.Cu") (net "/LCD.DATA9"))
 (segment (start 165.4 57.1) (end 166.582 55.918) (width 0.254) (layer "B.Cu") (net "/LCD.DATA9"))
 (segment (start 165.4 60) (end 165.4 57.1) (width 0.254) (layer "B.Cu") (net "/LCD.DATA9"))
 (segment (start 169.308 48.658) (end 167.945 47.295) (width 0.254) (layer "B.Cu") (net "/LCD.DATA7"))
 (segment (start 173 60) (end 169.308 56.308) (width 0.254) (layer "B.Cu") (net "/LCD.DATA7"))
 (segment (start 169.308 56.308) (end 169.308 48.658) (width 0.254) (layer "B.Cu") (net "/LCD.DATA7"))
 (segment (start 171.848 56.348) (end 171.848 48.658) (width 0.254) (layer "B.Cu") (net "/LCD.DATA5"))
 (segment (start 175.5 60) (end 171.848 56.348) (width 0.254) (layer "B.Cu") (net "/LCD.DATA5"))
 (segment (start 171.848 48.658) (end 170.485 47.295) (width 0.254) (layer "B.Cu") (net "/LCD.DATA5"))
 (segment (start 174.202 48.472) (end 173.025 47.295) (width 0.254) (layer "B.Cu") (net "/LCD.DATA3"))
 (segment (start 174.202 56.202) (end 174.202 48.472) (width 0.254) (layer "B.Cu") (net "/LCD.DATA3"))
 (segment (start 178 60) (end 174.202 56.202) (width 0.254) (layer "B.Cu") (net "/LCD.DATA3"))
 (segment (start 180.5 60) (end 176.742 56.242) (width 0.254) (layer "B.Cu") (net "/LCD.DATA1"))
 (segment (start 176.742 56.242) (end 176.742 48.472) (width 0.254) (layer "B.Cu") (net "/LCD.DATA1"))
 (segment (start 176.742 48.472) (end 175.565 47.295) (width 0.254) (layer "B.Cu") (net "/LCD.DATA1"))
 (segment (start 122.225 90.275) (end 122.225 98.095) (width 0.5) (layer "B.Cu") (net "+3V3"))
 (segment (start 121.25 88.75) (end 122.5 90) (width 0.5) (layer "B.Cu") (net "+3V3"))
 (segment (start 106.025 88.75) (end 121.25 88.75) (width 0.5) (layer "B.Cu") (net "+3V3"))
 (segment (start 122.5 90) (end 122.225 90.275) (width 0.5) (layer "B.Cu") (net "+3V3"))
 (segment (start 124.75 83.75) (end 125 84) (width 0.5) (layer "B.Cu") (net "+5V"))
 (segment (start 124.765 84.235) (end 124.765 95.555) (width 0.5) (layer "B.Cu") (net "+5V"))
 (segment (start 106.025 83.75) (end 124.75 83.75) (width 0.5) (layer "B.Cu") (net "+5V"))
 (segment (start 125 84) (end 124.765 84.235) (width 0.5) (layer "B.Cu") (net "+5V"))
 (segment (start 154 95.13547) (end 154 96.8) (width 0.254) (layer "B.Cu") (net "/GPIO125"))
 (segment (start 164.63547 84.5) (end 154 95.13547) (width 0.254) (layer "B.Cu") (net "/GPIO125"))
 (segment (start 154 96.8) (end 152.705 98.095) (width 0.254) (layer "B.Cu") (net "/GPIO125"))
 (segment (start 174.5 84.5) (end 164.63547 84.5) (width 0.254) (layer "B.Cu") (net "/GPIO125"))
 (segment (start 177 89.04) (end 177 84.5) (width 0.254) (layer "B.Cu") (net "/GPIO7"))
 (segment (start 170.485 95.555) (end 177 89.04) (width 0.254) (layer "B.Cu") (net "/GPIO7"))
 (segment (start 179.177 67.177) (end 179.177 58.677) (width 0.254) (layer "F.Cu") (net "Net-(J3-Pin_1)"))
 (segment (start 175.565 55.065) (end 175.565 49.835) (width 0.254) (layer "F.Cu") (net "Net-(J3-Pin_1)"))
 (segment (start 180.5 68.5) (end 179.177 67.177) (width 0.254) (layer "F.Cu") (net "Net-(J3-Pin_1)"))
 (segment (start 179.177 58.677) (end 175.565 55.065) (width 0.254) (layer "F.Cu") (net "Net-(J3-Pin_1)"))
 (segment (start 173 55) (end 173.025 54.975) (width 0.254) (layer "F.Cu") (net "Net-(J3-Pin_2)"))
 (segment (start 176.677 67.177) (end 176.677 58.677) (width 0.254) (layer "F.Cu") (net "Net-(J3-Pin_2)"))
 (segment (start 173.025 54.975) (end 173.025 49.835) (width 0.254) (layer "F.Cu") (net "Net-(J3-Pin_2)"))
 (segment (start 176.677 58.677) (end 173 55) (width 0.254) (layer "F.Cu") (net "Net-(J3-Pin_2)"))
 (segment (start 178 68.5) (end 176.677 67.177) (width 0.254) (layer "F.Cu") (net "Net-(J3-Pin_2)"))
 (segment (start 174.177 67.177) (end 174.177 58.677) (width 0.254) (layer "F.Cu") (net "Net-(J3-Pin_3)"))
 (segment (start 170.5 53) (end 170.485 52.985) (width 0.254) (layer "F.Cu") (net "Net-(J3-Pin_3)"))
 (segment (start 170.485 52.985) (end 170.485 49.835) (width 0.254) (layer "F.Cu") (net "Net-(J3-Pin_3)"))
 (segment (start 174.177 58.677) (end 170.5 55) (width 0.254) (layer "F.Cu") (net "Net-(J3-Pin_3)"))
 (segment (start 170.5 55) (end 170.5 53) (width 0.254) (layer "F.Cu") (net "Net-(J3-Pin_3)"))
 (segment (start 175.5 68.5) (end 174.177 67.177) (width 0.254) (layer "F.Cu") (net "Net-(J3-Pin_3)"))
 (segment (start 167.945 54.945) (end 167.945 49.835) (width 0.254) (layer "F.Cu") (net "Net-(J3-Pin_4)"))
 (segment (start 171.5 67) (end 171.5 58.5) (width 0.254) (layer "F.Cu") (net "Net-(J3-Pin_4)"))
 (segment (start 171.5 58.5) (end 167.945 54.945) (width 0.254) (layer "F.Cu") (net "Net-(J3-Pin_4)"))
 (segment (start 173 68.5) (end 171.5 67) (width 0.254) (layer "F.Cu") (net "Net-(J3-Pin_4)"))
 (segment (start 165.4 68.5) (end 164.223 67.323) (width 0.254) (layer "B.Cu") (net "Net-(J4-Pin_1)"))
 (segment (start 164.223 51.017) (end 165.405 49.835) (width 0.254) (layer "B.Cu") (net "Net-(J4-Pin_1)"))
 (segment (start 164.223 67.323) (end 164.223 51.017) (width 0.254) (layer "B.Cu") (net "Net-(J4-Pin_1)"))
 (segment (start 156.723 50.897) (end 157.785 49.835) (width 0.254) (layer "B.Cu") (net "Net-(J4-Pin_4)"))
 (segment (start 156.723 67.323) (end 156.723 50.897) (width 0.254) (layer "B.Cu") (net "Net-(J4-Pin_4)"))
 (segment (start 157.9 68.5) (end 156.723 67.323) (width 0.254) (layer "B.Cu") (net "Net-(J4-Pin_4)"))
 (segment (start 159.223 50.937) (end 160.325 49.835) (width 0.254) (layer "B.Cu") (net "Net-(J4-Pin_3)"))
 (segment (start 160.4 68.5) (end 159.223 67.323) (width 0.254) (layer "B.Cu") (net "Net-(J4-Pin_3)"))
 (segment (start 159.223 67.323) (end 159.223 50.937) (width 0.254) (layer "B.Cu") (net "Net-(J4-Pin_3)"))
 (segment (start 161.723 55.5) (end 161.723 50.977) (width 0.254) (layer "B.Cu") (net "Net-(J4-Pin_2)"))
 (segment (start 161.723 55.5) (end 161 55.5) (width 0.254) (layer "B.Cu") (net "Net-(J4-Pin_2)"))
 (segment (start 162.9 68.5) (end 161.723 67.323) (width 0.254) (layer "B.Cu") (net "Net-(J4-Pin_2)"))
 (segment (start 161.723 67.323) (end 161.723 55.5) (width 0.254) (layer "B.Cu") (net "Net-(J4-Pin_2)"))
 (segment (start 161.723 50.977) (end 162.865 49.835) (width 0.254) (layer "B.Cu") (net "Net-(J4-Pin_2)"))
 (segment (start 112.5 55) (end 114 53.5) (width 0.254) (layer "B.Cu") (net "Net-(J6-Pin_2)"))
 (segment (start 131 53.5) (end 132.5 52) (width 0.254) (layer "B.Cu") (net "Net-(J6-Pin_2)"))
 (segment (start 112.5 55.975) (end 112.5 55) (width 0.254) (layer "B.Cu") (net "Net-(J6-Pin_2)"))
 (segment (start 132.385 51.885) (end 132.385 49.835) (width 0.254) (layer "B.Cu") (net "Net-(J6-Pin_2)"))
 (segment (start 132.5 52) (end 132.385 51.885) (width 0.254) (layer "B.Cu") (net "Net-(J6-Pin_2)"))
 (segment (start 114 53.5) (end 131 53.5) (width 0.254) (layer "B.Cu") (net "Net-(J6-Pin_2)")))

